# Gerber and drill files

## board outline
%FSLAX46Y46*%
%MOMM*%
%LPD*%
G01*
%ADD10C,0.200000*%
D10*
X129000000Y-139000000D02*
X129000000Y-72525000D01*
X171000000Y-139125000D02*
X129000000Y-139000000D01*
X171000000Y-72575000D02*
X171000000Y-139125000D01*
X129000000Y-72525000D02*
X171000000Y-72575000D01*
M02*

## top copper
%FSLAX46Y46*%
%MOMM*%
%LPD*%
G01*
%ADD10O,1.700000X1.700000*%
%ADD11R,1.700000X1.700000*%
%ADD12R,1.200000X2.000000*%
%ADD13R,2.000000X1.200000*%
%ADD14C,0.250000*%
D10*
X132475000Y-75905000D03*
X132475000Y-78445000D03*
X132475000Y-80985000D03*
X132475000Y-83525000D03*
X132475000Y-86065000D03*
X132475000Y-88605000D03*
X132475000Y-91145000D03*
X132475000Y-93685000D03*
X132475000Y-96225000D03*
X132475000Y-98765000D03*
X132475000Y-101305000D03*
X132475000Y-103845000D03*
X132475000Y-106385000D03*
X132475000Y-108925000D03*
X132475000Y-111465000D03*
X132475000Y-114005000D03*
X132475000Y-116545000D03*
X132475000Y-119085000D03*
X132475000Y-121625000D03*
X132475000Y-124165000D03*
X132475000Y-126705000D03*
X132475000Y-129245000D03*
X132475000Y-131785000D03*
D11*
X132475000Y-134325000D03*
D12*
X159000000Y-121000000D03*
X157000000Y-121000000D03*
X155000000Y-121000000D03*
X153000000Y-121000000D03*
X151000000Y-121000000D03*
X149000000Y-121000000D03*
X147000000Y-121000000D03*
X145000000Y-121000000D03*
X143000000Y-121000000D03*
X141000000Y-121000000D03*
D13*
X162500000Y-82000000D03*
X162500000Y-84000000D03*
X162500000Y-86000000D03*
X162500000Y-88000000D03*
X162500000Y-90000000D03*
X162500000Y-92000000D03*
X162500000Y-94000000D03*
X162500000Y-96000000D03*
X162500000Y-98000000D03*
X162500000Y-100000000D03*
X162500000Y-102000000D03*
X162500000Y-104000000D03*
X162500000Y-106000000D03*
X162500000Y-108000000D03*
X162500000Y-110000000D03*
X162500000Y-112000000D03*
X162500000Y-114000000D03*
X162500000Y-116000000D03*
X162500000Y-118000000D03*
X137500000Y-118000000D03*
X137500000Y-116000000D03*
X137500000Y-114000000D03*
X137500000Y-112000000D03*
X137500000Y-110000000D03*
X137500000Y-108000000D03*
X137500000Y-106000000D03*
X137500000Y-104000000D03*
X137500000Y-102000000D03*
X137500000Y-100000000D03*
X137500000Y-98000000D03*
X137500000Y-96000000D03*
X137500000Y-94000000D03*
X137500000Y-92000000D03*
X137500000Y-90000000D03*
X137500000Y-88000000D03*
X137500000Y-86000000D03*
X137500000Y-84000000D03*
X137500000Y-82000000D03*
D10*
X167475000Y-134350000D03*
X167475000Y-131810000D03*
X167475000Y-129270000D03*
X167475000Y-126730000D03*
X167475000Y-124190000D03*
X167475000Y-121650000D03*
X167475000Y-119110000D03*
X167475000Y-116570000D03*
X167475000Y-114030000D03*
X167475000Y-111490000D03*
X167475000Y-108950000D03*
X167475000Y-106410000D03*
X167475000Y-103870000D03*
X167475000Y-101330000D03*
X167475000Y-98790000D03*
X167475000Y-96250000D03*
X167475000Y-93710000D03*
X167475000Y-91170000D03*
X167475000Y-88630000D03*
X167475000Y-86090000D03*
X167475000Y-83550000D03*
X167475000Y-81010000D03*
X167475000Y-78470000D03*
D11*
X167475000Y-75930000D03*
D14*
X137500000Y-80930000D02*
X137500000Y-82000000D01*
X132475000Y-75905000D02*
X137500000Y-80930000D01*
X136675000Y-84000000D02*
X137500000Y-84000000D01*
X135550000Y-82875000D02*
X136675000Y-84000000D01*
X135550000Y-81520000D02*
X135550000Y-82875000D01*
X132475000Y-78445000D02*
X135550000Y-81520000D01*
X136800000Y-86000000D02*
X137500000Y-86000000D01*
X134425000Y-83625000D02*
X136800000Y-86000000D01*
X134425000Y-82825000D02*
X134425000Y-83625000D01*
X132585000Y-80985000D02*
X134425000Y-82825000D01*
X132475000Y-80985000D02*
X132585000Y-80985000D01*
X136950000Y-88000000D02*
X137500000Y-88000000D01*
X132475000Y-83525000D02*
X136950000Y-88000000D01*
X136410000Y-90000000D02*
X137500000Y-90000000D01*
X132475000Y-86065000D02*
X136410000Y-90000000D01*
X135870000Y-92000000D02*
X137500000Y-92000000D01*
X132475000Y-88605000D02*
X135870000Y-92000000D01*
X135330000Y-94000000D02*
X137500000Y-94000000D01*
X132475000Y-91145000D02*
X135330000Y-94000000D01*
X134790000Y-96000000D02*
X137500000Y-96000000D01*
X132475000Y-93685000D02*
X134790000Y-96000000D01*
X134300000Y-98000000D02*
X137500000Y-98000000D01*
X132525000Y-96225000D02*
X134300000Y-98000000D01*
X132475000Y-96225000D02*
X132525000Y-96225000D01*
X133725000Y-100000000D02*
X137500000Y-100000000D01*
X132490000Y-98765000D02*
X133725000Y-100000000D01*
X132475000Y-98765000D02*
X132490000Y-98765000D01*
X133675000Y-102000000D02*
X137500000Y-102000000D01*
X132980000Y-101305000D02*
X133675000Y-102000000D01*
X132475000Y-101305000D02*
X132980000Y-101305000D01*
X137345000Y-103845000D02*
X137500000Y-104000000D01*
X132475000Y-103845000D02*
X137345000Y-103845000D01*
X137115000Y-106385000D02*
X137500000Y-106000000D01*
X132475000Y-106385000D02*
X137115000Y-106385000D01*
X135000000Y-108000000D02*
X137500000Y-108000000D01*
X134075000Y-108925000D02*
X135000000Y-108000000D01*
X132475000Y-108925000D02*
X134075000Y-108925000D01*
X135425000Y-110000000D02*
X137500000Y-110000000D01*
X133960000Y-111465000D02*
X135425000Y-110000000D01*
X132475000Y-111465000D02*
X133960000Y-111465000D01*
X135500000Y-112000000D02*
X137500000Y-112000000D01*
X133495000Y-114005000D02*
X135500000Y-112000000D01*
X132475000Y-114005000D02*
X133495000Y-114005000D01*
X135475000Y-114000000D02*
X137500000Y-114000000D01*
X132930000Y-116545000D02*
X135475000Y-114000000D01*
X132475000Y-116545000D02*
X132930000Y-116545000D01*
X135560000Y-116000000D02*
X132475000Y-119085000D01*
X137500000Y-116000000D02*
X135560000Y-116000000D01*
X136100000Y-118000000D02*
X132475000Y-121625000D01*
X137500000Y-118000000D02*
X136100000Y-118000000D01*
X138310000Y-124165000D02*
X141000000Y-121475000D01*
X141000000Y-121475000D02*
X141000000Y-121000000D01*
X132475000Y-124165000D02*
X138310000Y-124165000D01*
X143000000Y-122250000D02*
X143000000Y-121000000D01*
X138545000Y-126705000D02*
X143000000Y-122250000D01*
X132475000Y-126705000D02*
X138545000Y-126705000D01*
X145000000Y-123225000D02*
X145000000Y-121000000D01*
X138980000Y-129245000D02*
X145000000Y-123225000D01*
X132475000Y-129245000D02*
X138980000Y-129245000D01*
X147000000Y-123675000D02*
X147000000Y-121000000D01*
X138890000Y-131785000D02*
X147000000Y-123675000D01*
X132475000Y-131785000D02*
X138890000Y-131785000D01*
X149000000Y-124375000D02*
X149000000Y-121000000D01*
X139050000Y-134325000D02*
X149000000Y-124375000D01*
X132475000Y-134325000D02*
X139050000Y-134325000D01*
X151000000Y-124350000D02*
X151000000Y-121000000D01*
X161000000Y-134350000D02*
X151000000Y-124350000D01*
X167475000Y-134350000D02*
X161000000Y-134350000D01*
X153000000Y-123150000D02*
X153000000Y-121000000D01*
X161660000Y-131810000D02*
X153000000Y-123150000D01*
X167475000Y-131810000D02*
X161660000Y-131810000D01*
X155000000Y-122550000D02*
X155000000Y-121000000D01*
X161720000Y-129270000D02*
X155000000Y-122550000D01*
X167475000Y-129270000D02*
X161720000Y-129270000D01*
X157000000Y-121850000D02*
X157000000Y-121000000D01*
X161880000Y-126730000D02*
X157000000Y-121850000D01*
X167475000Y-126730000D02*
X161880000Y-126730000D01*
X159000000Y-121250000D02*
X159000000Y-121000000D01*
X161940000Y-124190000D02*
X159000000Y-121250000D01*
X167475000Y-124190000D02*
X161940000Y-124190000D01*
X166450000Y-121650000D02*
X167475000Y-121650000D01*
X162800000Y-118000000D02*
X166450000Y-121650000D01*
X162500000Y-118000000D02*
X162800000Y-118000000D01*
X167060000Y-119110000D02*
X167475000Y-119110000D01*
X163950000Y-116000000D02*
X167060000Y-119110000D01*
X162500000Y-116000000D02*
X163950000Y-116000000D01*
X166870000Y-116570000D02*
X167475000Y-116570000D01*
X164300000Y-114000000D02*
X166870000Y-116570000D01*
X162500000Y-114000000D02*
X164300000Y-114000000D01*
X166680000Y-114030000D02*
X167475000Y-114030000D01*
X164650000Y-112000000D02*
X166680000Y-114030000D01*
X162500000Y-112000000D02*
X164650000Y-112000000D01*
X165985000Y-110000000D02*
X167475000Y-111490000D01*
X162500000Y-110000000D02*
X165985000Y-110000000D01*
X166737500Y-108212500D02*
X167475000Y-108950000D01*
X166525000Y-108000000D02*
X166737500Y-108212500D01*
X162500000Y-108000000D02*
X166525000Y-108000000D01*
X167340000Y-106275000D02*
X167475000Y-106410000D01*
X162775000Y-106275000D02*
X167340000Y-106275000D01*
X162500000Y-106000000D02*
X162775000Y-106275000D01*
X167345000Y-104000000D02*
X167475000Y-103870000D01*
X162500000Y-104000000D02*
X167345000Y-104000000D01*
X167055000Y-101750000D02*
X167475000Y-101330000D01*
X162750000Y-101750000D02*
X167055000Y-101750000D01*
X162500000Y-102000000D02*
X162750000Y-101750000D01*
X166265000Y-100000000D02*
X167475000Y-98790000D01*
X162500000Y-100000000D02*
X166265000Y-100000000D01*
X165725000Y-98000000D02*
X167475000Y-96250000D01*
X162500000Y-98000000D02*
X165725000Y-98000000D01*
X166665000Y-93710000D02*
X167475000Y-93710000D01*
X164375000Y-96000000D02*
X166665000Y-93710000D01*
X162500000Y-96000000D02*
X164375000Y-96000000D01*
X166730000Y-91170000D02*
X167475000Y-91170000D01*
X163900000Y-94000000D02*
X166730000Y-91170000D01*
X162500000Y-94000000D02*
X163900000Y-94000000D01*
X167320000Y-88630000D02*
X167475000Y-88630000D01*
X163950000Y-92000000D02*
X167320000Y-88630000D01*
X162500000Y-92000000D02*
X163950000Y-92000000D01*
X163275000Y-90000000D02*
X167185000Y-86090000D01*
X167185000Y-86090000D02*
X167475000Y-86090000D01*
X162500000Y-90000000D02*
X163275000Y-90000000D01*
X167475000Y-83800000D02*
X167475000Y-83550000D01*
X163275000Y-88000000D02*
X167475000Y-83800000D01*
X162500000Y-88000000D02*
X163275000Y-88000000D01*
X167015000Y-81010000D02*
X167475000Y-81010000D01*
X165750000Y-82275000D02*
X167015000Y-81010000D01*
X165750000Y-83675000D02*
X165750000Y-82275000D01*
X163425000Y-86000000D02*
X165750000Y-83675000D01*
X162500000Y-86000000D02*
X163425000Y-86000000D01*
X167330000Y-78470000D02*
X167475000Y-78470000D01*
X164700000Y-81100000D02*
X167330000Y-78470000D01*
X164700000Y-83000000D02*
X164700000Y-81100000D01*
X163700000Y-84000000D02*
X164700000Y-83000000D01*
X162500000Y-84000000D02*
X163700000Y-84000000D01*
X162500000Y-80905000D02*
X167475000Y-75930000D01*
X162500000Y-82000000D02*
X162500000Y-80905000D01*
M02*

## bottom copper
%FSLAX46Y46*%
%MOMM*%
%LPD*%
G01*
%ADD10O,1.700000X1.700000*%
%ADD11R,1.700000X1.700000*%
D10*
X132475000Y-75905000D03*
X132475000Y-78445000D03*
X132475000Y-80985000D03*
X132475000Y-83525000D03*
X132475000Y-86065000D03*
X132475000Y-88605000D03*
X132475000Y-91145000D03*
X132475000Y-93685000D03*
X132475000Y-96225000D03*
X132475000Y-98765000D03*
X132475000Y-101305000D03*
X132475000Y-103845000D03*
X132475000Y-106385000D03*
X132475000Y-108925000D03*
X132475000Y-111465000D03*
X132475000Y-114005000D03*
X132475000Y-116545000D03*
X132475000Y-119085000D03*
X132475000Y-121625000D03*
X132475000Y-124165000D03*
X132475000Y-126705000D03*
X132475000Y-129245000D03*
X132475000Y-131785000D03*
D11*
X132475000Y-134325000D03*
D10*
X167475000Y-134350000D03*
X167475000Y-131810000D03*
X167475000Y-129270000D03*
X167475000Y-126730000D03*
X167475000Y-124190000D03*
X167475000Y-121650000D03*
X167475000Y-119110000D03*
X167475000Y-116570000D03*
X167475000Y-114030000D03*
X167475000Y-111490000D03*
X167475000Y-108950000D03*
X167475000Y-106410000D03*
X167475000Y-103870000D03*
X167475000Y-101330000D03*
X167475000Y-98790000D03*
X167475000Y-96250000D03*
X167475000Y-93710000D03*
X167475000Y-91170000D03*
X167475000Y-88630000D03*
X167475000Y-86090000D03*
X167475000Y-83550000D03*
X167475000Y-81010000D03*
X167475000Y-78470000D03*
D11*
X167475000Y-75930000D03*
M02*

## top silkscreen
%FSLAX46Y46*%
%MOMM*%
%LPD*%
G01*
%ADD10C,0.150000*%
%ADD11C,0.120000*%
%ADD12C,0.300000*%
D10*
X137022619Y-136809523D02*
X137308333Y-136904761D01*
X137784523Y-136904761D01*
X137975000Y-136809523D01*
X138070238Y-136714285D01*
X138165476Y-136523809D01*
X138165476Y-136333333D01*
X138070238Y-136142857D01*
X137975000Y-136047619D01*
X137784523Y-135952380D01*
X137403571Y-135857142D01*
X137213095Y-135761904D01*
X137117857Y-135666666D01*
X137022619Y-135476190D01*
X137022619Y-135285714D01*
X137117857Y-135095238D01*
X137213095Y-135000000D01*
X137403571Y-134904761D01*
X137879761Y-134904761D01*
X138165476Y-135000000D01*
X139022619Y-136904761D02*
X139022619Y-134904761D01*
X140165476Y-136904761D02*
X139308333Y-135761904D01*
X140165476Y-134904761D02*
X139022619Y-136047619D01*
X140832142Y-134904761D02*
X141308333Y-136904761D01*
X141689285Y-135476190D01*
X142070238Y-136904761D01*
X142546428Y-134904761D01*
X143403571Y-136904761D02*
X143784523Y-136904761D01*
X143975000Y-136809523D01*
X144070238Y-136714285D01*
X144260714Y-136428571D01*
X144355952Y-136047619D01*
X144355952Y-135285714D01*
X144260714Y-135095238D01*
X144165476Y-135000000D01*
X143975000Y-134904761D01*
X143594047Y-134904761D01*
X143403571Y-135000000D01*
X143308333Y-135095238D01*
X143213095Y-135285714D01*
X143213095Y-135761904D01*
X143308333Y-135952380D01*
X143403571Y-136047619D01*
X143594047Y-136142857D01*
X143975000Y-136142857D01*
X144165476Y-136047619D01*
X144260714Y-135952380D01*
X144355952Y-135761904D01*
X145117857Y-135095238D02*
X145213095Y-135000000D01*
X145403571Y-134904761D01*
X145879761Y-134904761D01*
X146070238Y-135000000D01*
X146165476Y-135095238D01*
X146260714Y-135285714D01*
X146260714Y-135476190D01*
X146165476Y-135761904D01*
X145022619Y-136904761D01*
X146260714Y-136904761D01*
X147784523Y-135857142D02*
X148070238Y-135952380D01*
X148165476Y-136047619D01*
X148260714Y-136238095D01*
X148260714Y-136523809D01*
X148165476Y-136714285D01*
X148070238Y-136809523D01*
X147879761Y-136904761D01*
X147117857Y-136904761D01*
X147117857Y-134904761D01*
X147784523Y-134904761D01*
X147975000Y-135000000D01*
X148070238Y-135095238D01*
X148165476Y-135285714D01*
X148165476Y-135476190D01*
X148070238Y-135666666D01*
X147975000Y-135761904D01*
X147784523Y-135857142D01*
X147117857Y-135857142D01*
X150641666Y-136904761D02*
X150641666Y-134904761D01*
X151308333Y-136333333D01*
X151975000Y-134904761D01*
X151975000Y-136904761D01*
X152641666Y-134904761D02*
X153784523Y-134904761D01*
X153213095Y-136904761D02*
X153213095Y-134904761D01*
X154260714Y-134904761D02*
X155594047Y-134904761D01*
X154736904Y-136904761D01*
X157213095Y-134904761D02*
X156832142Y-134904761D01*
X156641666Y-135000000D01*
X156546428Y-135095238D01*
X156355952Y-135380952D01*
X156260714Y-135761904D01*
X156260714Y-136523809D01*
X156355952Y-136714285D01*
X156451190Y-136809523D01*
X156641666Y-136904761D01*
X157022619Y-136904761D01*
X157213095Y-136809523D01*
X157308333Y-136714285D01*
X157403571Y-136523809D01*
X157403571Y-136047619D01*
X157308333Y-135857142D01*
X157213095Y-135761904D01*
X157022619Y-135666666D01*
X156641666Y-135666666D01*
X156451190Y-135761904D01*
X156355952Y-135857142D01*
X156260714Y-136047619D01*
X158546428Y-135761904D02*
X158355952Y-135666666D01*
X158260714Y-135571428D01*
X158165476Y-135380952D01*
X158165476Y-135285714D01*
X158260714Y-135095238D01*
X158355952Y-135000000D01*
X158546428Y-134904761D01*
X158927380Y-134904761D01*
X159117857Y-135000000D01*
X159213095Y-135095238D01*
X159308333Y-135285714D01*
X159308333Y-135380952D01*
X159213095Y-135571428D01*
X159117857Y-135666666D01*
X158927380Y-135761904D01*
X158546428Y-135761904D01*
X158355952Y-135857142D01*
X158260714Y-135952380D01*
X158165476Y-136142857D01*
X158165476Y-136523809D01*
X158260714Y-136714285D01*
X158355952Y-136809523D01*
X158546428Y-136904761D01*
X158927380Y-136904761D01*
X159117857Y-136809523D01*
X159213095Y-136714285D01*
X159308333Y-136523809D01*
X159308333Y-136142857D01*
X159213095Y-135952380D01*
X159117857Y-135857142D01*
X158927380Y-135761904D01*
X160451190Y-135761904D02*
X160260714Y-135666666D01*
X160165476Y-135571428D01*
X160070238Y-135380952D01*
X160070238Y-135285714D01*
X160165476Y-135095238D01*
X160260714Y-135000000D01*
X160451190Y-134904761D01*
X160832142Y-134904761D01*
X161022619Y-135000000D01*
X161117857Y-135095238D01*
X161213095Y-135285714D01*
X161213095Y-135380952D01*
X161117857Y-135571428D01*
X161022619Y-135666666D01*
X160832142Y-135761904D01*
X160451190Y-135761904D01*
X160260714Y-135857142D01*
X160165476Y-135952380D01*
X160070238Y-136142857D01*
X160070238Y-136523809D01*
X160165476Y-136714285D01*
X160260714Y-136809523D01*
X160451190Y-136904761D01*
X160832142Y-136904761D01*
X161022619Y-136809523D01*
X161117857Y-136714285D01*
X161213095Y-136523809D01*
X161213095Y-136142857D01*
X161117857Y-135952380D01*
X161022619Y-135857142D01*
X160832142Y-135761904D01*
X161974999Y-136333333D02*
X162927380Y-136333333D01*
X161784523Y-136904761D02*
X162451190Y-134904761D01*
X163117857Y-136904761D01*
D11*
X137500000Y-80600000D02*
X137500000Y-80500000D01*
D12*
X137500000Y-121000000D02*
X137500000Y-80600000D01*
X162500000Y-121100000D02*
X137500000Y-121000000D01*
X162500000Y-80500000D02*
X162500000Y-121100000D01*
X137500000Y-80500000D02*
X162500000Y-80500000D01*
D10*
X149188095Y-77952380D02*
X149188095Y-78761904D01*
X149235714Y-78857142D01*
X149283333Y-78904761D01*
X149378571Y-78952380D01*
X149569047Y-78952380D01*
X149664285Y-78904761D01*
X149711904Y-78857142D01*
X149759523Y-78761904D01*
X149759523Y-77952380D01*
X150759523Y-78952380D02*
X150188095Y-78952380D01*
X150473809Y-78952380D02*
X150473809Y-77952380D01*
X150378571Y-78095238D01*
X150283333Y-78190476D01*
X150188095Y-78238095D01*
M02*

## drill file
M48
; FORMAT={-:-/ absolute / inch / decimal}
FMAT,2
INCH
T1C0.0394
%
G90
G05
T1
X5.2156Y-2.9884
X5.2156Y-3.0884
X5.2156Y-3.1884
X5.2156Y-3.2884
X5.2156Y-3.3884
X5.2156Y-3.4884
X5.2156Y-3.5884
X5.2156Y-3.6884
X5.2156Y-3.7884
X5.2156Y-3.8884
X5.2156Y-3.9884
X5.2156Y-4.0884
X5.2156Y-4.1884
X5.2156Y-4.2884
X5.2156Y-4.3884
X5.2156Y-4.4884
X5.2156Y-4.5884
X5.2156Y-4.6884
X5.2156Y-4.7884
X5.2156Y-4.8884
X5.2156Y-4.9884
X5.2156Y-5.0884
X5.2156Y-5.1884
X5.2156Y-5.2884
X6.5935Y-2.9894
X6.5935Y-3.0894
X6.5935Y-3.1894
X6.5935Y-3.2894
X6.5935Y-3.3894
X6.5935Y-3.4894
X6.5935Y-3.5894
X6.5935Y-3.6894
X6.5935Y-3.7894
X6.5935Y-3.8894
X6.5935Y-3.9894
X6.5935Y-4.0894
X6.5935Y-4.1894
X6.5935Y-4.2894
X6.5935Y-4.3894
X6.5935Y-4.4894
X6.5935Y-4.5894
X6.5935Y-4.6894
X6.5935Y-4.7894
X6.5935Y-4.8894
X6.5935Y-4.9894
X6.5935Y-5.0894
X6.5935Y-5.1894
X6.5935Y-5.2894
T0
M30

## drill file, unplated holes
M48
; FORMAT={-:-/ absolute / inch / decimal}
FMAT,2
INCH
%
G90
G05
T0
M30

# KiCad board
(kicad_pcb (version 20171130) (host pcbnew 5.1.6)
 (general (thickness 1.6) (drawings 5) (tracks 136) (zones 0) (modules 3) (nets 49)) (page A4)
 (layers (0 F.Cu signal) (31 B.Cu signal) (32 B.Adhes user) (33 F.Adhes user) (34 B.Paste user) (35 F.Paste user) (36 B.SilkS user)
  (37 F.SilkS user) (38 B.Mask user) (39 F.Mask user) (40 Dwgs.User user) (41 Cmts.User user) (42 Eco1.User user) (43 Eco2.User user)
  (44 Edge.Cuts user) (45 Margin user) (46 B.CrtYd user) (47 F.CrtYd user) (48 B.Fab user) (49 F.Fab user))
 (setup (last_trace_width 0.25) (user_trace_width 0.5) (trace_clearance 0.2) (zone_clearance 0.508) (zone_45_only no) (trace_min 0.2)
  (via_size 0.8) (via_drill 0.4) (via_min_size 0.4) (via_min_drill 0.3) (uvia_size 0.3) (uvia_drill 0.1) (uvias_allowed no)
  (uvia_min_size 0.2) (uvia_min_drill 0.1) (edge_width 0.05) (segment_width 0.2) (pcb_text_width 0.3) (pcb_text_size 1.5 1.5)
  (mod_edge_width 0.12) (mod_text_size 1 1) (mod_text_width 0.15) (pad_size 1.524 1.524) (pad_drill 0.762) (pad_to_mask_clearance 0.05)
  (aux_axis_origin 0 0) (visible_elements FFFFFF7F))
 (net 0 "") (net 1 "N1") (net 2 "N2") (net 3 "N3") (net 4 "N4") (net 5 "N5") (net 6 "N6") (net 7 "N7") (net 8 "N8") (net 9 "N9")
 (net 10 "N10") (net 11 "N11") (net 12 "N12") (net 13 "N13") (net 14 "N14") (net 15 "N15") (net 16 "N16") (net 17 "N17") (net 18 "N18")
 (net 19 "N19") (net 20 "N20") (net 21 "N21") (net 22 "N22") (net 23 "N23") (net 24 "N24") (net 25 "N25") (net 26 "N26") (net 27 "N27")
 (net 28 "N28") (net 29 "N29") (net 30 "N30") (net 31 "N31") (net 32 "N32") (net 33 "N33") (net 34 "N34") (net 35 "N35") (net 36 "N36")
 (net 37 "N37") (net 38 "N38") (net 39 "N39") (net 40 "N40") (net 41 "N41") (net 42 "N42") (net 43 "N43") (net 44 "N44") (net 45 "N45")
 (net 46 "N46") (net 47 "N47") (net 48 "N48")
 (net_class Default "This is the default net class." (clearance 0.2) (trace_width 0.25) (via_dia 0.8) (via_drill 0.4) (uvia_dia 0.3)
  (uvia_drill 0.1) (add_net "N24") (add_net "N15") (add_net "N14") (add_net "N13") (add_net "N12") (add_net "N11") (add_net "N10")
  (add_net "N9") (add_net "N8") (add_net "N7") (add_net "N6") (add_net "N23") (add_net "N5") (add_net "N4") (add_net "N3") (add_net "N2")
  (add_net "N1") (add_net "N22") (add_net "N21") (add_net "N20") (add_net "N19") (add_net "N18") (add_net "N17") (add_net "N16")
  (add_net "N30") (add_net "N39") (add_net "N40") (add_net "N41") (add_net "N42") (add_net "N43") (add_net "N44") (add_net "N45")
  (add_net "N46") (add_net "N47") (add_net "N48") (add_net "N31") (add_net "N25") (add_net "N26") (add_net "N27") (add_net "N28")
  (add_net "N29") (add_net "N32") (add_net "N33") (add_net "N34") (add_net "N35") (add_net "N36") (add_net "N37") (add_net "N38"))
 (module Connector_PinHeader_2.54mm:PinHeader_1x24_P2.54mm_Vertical (layer B.Cu) (at 132.475 134.325)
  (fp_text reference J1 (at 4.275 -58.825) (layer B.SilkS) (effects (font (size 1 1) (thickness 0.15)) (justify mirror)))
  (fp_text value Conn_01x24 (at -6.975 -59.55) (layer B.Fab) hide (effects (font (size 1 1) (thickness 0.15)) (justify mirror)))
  (pad 24 thru_hole oval (at 0 -58.42) (size 1.7 1.7) (drill 1) (layers *.Cu *.Mask) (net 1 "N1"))
  (pad 23 thru_hole oval (at 0 -55.88) (size 1.7 1.7) (drill 1) (layers *.Cu *.Mask) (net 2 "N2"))
  (pad 22 thru_hole oval (at 0 -53.34) (size 1.7 1.7) (drill 1) (layers *.Cu *.Mask) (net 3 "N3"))
  (pad 21 thru_hole oval (at 0 -50.8) (size 1.7 1.7) (drill 1) (layers *.Cu *.Mask) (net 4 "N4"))
  (pad 20 thru_hole oval (at 0 -48.26) (size 1.7 1.7) (drill 1) (layers *.Cu *.Mask) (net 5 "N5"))
  (pad 19 thru_hole oval (at 0 -45.72) (size 1.7 1.7) (drill 1) (layers *.Cu *.Mask) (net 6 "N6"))
  (pad 18 thru_hole oval (at 0 -43.18) (size 1.7 1.7) (drill 1) (layers *.Cu *.Mask) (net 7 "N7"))
  (pad 17 thru_hole oval (at 0 -40.64) (size 1.7 1.7) (drill 1) (layers *.Cu *.Mask) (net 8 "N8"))
  (pad 16 thru_hole oval (at 0 -38.1) (size 1.7 1.7) (drill 1) (layers *.Cu *.Mask) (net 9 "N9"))
  (pad 15 thru_hole oval (at 0 -35.56) (size 1.7 1.7) (drill 1) (layers *.Cu *.Mask) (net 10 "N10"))
  (pad 14 thru_hole oval (at 0 -33.02) (size 1.7 1.7) (drill 1) (layers *.Cu *.Mask) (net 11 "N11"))
  (pad 13 thru_hole oval (at 0 -30.48) (size 1.7 1.7) (drill 1) (layers *.Cu *.Mask) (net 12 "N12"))
  (pad 12 thru_hole oval (at 0 -27.94) (size 1.7 1.7) (drill 1) (layers *.Cu *.Mask) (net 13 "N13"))
  (pad 11 thru_hole oval (at 0 -25.4) (size 1.7 1.7) (drill 1) (layers *.Cu *.Mask) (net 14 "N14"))
  (pad 10 thru_hole oval (at 0 -22.86) (size 1.7 1.7) (drill 1) (layers *.Cu *.Mask) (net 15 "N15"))
  (pad 9 thru_hole oval (at 0 -20.32) (size 1.7 1.7) (drill 1) (layers *.Cu *.Mask) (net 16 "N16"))
  (pad 8 thru_hole oval (at 0 -17.78) (size 1.7 1.7) (drill 1) (layers *.Cu *.Mask) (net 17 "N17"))
  (pad 7 thru_hole oval (at 0 -15.24) (size 1.7 1.7) (drill 1) (layers *.Cu *.Mask) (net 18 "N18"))
  (pad 6 thru_hole oval (at 0 -12.7) (size 1.7 1.7) (drill 1) (layers *.Cu *.Mask) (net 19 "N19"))
  (pad 5 thru_hole oval (at 0 -10.16) (size 1.7 1.7) (drill 1) (layers *.Cu *.Mask) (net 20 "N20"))
  (pad 4 thru_hole oval (at 0 -7.62) (size 1.7 1.7) (drill 1) (layers *.Cu *.Mask) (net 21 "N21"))
  (pad 3 thru_hole oval (at 0 -5.08) (size 1.7 1.7) (drill 1) (layers *.Cu *.Mask) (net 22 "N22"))
  (pad 2 thru_hole oval (at 0 -2.54) (size 1.7 1.7) (drill 1) (layers *.Cu *.Mask) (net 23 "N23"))
  (pad 1 thru_hole rect (at 0 0) (size 1.7 1.7) (drill 1) (layers *.Cu *.Mask) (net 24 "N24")))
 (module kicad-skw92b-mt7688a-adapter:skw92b (layer F.Cu) (at 150 100)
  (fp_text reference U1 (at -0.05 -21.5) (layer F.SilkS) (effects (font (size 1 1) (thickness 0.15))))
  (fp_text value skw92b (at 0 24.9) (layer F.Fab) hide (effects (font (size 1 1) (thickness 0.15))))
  (fp_line (start -12.5 -19.4) (end -12.5 -19.5) (layer F.SilkS) (width 0.12))
  (fp_line (start -12.5 21) (end -12.5 -19.4) (layer F.SilkS) (width 0.3))
  (fp_line (start 12.5 21.1) (end -12.5 21) (layer F.SilkS) (width 0.3))
  (fp_line (start 12.5 -19.5) (end 12.5 21.1) (layer F.SilkS) (width 0.3))
  (fp_line (start -12.5 -19.5) (end 12.5 -19.5) (layer F.SilkS) (width 0.3))
  (pad 29 smd rect (at 9 21) (size 1.2 2) (layers F.Cu F.Paste F.Mask) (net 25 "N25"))
  (pad 28 smd rect (at 7 21) (size 1.2 2) (layers F.Cu F.Paste F.Mask) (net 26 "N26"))
  (pad 27 smd rect (at 5 21) (size 1.2 2) (layers F.Cu F.Paste F.Mask) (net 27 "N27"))
  (pad 26 smd rect (at 3 21) (size 1.2 2) (layers F.Cu F.Paste F.Mask) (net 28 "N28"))
  (pad 25 smd rect (at 1 21) (size 1.2 2) (layers F.Cu F.Paste F.Mask) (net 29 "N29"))
  (pad 24 smd rect (at -1 21) (size 1.2 2) (layers F.Cu F.Paste F.Mask) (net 24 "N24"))
  (pad 23 smd rect (at -3 21) (size 1.2 2) (layers F.Cu F.Paste F.Mask) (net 23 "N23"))
  (pad 22 smd rect (at -5 21) (size 1.2 2) (layers F.Cu F.Paste F.Mask) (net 22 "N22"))
  (pad 21 smd rect (at -7 21) (size 1.2 2) (layers F.Cu F.Paste F.Mask) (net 21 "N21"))
  (pad 20 smd rect (at -9 21) (size 1.2 2) (layers F.Cu F.Paste F.Mask) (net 20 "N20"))
  (pad 48 smd rect (at 12.5 -18) (size 2 1.2) (layers F.Cu F.Paste F.Mask) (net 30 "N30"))
  (pad 47 smd rect (at 12.5 -16) (size 2 1.2) (layers F.Cu F.Paste F.Mask) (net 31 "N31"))
  (pad 46 smd rect (at 12.5 -14) (size 2 1.2) (layers F.Cu F.Paste F.Mask) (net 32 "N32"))
  (pad 45 smd rect (at 12.5 -12) (size 2 1.2) (layers F.Cu F.Paste F.Mask) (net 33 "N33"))
  (pad 44 smd rect (at 12.5 -10) (size 2 1.2) (layers F.Cu F.Paste F.Mask) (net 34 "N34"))
  (pad 43 smd rect (at 12.5 -8) (size 2 1.2) (layers F.Cu F.Paste F.Mask) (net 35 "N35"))
  (pad 42 smd rect (at 12.5 -6) (size 2 1.2) (layers F.Cu F.Paste F.Mask) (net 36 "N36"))
  (pad 41 smd rect (at 12.5 -4) (size 2 1.2) (layers F.Cu F.Paste F.Mask) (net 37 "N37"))
  (pad 40 smd rect (at 12.5 -2) (size 2 1.2) (layers F.Cu F.Paste F.Mask) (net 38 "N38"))
  (pad 39 smd rect (at 12.5 0) (size 2 1.2) (layers F.Cu F.Paste F.Mask) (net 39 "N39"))
  (pad 38 smd rect (at 12.5 2) (size 2 1.2) (layers F.Cu F.Paste F.Mask) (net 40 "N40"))
  (pad 37 smd rect (at 12.5 4) (size 2 1.2) (layers F.Cu F.Paste F.Mask) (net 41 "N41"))
  (pad 36 smd rect (at 12.5 6) (size 2 1.2) (layers F.Cu F.Paste F.Mask) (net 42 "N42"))
  (pad 35 smd rect (at 12.5 8) (size 2 1.2) (layers F.Cu F.Paste F.Mask) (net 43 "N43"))
  (pad 34 smd rect (at 12.5 10) (size 2 1.2) (layers F.Cu F.Paste F.Mask) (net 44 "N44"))
  (pad 33 smd rect (at 12.5 12) (size 2 1.2) (layers F.Cu F.Paste F.Mask) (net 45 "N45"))
  (pad 32 smd rect (at 12.5 14) (size 2 1.2) (layers F.Cu F.Paste F.Mask) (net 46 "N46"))
  (pad 31 smd rect (at 12.5 16) (size 2 1.2) (layers F.Cu F.Paste F.Mask) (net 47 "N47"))
  (pad 30 smd rect (at 12.5 18) (size 2 1.2) (layers F.Cu F.Paste F.Mask) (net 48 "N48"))
  (pad 19 smd rect (at -12.5 18) (size 2 1.2) (layers F.Cu F.Paste F.Mask) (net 19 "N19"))
  (pad 18 smd rect (at -12.5 16) (size 2 1.2) (layers F.Cu F.Paste F.Mask) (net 18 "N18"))
  (pad 17 smd rect (at -12.5 14) (size 2 1.2) (layers F.Cu F.Paste F.Mask) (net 17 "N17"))
  (pad 16 smd rect (at -12.5 12) (size 2 1.2) (layers F.Cu F.Paste F.Mask) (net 16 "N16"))
  (pad 15 smd rect (at -12.5 10) (size 2 1.2) (layers F.Cu F.Paste F.Mask) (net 15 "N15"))
  (pad 14 smd rect (at -12.5 8) (size 2 1.2) (layers F.Cu F.Paste F.Mask) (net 14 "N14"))
  (pad 13 smd rect (at -12.5 6) (size 2 1.2) (layers F.Cu F.Paste F.Mask) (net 13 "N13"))
  (pad 12 smd rect (at -12.5 4) (size 2 1.2) (layers F.Cu F.Paste F.Mask) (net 12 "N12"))
  (pad 11 smd rect (at -12.5 2) (size 2 1.2) (layers F.Cu F.Paste F.Mask) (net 11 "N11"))
  (pad 10 smd rect (at -12.5 0) (size 2 1.2) (layers F.Cu F.Paste F.Mask) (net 10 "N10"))
  (pad 9 smd rect (at -12.5 -2) (size 2 1.2) (layers F.Cu F.Paste F.Mask) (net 9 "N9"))
  (pad 8 smd rect (at -12.5 -4) (size 2 1.2) (layers F.Cu F.Paste F.Mask) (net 8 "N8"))
  (pad 7 smd rect (at -12.5 -6) (size 2 1.2) (layers F.Cu F.Paste F.Mask) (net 7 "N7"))
  (pad 6 smd rect (at -12.5 -8) (size 2 1.2) (layers F.Cu F.Paste F.Mask) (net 6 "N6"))
  (pad 5 smd rect (at -12.5 -10) (size 2 1.2) (layers F.Cu F.Paste F.Mask) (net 5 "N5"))
  (pad 4 smd rect (at -12.5 -12) (size 2 1.2) (layers F.Cu F.Paste F.Mask) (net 4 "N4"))
  (pad 3 smd rect (at -12.5 -14) (size 2 1.2) (layers F.Cu F.Paste F.Mask) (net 3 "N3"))
  (pad 2 smd rect (at -12.5 -16) (size 2 1.2) (layers F.Cu F.Paste F.Mask) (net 2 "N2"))
  (pad 1 smd rect (at -12.5 -18) (size 2 1.2) (layers F.Cu F.Paste F.Mask) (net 1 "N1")))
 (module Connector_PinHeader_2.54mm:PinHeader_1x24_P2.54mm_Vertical (layer B.Cu) (at 167.475 75.93 180)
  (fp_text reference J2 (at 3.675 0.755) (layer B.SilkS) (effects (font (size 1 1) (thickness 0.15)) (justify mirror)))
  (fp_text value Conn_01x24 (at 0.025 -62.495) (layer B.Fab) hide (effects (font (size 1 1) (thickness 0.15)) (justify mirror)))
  (pad 24 thru_hole oval (at 0 -58.42 180) (size 1.7 1.7) (drill 1) (layers *.Cu *.Mask) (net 29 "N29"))
  (pad 23 thru_hole oval (at 0 -55.88 180) (size 1.7 1.7) (drill 1) (layers *.Cu *.Mask) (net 28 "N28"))
  (pad 22 thru_hole oval (at 0 -53.34 180) (size 1.7 1.7) (drill 1) (layers *.Cu *.Mask) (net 27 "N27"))
  (pad 21 thru_hole oval (at 0 -50.8 180) (size 1.7 1.7) (drill 1) (layers *.Cu *.Mask) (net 26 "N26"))
  (pad 20 thru_hole oval (at 0 -48.26 180) (size 1.7 1.7) (drill 1) (layers *.Cu *.Mask) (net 25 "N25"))
  (pad 19 thru_hole oval (at 0 -45.72 180) (size 1.7 1.7) (drill 1) (layers *.Cu *.Mask) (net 48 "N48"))
  (pad 18 thru_hole oval (at 0 -43.18 180) (size 1.7 1.7) (drill 1) (layers *.Cu *.Mask) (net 47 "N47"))
  (pad 17 thru_hole oval (at 0 -40.64 180) (size 1.7 1.7) (drill 1) (layers *.Cu *.Mask) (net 46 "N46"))
  (pad 16 thru_hole oval (at 0 -38.1 180) (size 1.7 1.7) (drill 1) (layers *.Cu *.Mask) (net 45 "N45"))
  (pad 15 thru_hole oval (at 0 -35.56 180) (size 1.7 1.7) (drill 1) (layers *.Cu *.Mask) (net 44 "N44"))
  (pad 14 thru_hole oval (at 0 -33.02 180) (size 1.7 1.7) (drill 1) (layers *.Cu *.Mask) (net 43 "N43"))
  (pad 13 thru_hole oval (at 0 -30.48 180) (size 1.7 1.7) (drill 1) (layers *.Cu *.Mask) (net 42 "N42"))
  (pad 12 thru_hole oval (at 0 -27.94 180) (size 1.7 1.7) (drill 1) (layers *.Cu *.Mask) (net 41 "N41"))
  (pad 11 thru_hole oval (at 0 -25.4 180) (size 1.7 1.7) (drill 1) (layers *.Cu *.Mask) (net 40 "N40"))
  (pad 10 thru_hole oval (at 0 -22.86 180) (size 1.7 1.7) (drill 1) (layers *.Cu *.Mask) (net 39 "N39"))
  (pad 9 thru_hole oval (at 0 -20.32 180) (size 1.7 1.7) (drill 1) (layers *.Cu *.Mask) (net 38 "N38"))
  (pad 8 thru_hole oval (at 0 -17.78 180) (size 1.7 1.7) (drill 1) (layers *.Cu *.Mask) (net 37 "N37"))
  (pad 7 thru_hole oval (at 0 -15.24 180) (size 1.7 1.7) (drill 1) (layers *.Cu *.Mask) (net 36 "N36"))
  (pad 6 thru_hole oval (at 0 -12.7 180) (size 1.7 1.7) (drill 1) (layers *.Cu *.Mask) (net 35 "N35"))
  (pad 5 thru_hole oval (at 0 -10.16 180) (size 1.7 1.7) (drill 1) (layers *.Cu *.Mask) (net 34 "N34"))
  (pad 4 thru_hole oval (at 0 -7.62 180) (size 1.7 1.7) (drill 1) (layers *.Cu *.Mask) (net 33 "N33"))
  (pad 3 thru_hole oval (at 0 -5.08 180) (size 1.7 1.7) (drill 1) (layers *.Cu *.Mask) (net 32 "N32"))
  (pad 2 thru_hole oval (at 0 -2.54 180) (size 1.7 1.7) (drill 1) (layers *.Cu *.Mask) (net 31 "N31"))
  (pad 1 thru_hole rect (at 0 0 180) (size 1.7 1.7) (drill 1) (layers *.Cu *.Mask) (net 30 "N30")))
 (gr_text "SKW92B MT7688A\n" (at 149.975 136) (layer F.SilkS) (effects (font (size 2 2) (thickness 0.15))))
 (gr_line (start 129 139) (end 129 72.525) (layer Edge.Cuts) (width 0.2))
 (gr_line (start 171 139.125) (end 129 139) (layer Edge.Cuts) (width 0.2))
 (gr_line (start 171 72.575) (end 171 139.125) (layer Edge.Cuts) (width 0.2))
 (gr_line (start 129 72.525) (end 171 72.575) (layer Edge.Cuts) (width 0.2))
 (segment (start 137.5 80.93) (end 137.5 82) (width 0.25) (layer F.Cu) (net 1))
 (segment (start 132.475 75.905) (end 137.5 80.93) (width 0.25) (layer F.Cu) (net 1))
 (segment (start 136.675 84) (end 137.5 84) (width 0.25) (layer F.Cu) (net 2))
 (segment (start 135.55 82.875) (end 136.675 84) (width 0.25) (layer F.Cu) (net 2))
 (segment (start 135.55 81.52) (end 135.55 82.875) (width 0.25) (layer F.Cu) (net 2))
 (segment (start 132.475 78.445) (end 135.55 81.52) (width 0.25) (layer F.Cu) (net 2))
 (segment (start 136.8 86) (end 137.5 86) (width 0.25) (layer F.Cu) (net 3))
 (segment (start 134.425 83.625) (end 136.8 86) (width 0.25) (layer F.Cu) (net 3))
 (segment (start 134.425 82.825) (end 134.425 83.625) (width 0.25) (layer F.Cu) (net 3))
 (segment (start 132.585 80.985) (end 134.425 82.825) (width 0.25) (layer F.Cu) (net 3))
 (segment (start 132.475 80.985) (end 132.585 80.985) (width 0.25) (layer F.Cu) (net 3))
 (segment (start 136.95 88) (end 137.5 88) (width 0.25) (layer F.Cu) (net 4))
 (segment (start 132.475 83.525) (end 136.95 88) (width 0.25) (layer F.Cu) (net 4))
 (segment (start 136.41 90) (end 137.5 90) (width 0.25) (layer F.Cu) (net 5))
 (segment (start 132.475 86.065) (end 136.41 90) (width 0.25) (layer F.Cu) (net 5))
 (segment (start 135.87 92) (end 137.5 92) (width 0.25) (layer F.Cu) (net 6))
 (segment (start 132.475 88.605) (end 135.87 92) (width 0.25) (layer F.Cu) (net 6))
 (segment (start 135.33 94) (end 137.5 94) (width 0.25) (layer F.Cu) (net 7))
 (segment (start 132.475 91.145) (end 135.33 94) (width 0.25) (layer F.Cu) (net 7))
 (segment (start 134.79 96) (end 137.5 96) (width 0.25) (layer F.Cu) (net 8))
 (segment (start 132.475 93.685) (end 134.79 96) (width 0.25) (layer F.Cu) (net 8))
 (segment (start 134.3 98) (end 137.5 98) (width 0.25) (layer F.Cu) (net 9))
 (segment (start 132.525 96.225) (end 134.3 98) (width 0.25) (layer F.Cu) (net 9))
 (segment (start 132.475 96.225) (end 132.525 96.225) (width 0.25) (layer F.Cu) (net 9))
 (segment (start 133.725 100) (end 137.5 100) (width 0.25) (layer F.Cu) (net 10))
 (segment (start 132.49 98.765) (end 133.725 100) (width 0.25) (layer F.Cu) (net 10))
 (segment (start 132.475 98.765) (end 132.49 98.765) (width 0.25) (layer F.Cu) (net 10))
 (segment (start 133.675 102) (end 137.5 102) (width 0.25) (layer F.Cu) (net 11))
 (segment (start 132.98 101.305) (end 133.675 102) (width 0.25) (layer F.Cu) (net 11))
 (segment (start 132.475 101.305) (end 132.98 101.305) (width 0.25) (layer F.Cu) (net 11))
 (segment (start 137.345 103.845) (end 137.5 104) (width 0.25) (layer F.Cu) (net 12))
 (segment (start 132.475 103.845) (end 137.345 103.845) (width 0.25) (layer F.Cu) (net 12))
 (segment (start 137.115 106.385) (end 137.5 106) (width 0.25) (layer F.Cu) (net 13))
 (segment (start 132.475 106.385) (end 137.115 106.385) (width 0.25) (layer F.Cu) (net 13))
 (segment (start 135 108) (end 137.5 108) (width 0.25) (layer F.Cu) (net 14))
 (segment (start 134.075 108.925) (end 135 108) (width 0.25) (layer F.Cu) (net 14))
 (segment (start 132.475 108.925) (end 134.075 108.925) (width 0.25) (layer F.Cu) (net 14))
 (segment (start 135.425 110) (end 137.5 110) (width 0.25) (layer F.Cu) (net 15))
 (segment (start 133.96 111.465) (end 135.425 110) (width 0.25) (layer F.Cu) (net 15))
 (segment (start 132.475 111.465) (end 133.96 111.465) (width 0.25) (layer F.Cu) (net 15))
 (segment (start 135.5 112) (end 137.5 112) (width 0.25) (layer F.Cu) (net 16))
 (segment (start 133.495 114.005) (end 135.5 112) (width 0.25) (layer F.Cu) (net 16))
 (segment (start 132.475 114.005) (end 133.495 114.005) (width 0.25) (layer F.Cu) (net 16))
 (segment (start 135.475 114) (end 137.5 114) (width 0.25) (layer F.Cu) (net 17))
 (segment (start 132.93 116.545) (end 135.475 114) (width 0.25) (layer F.Cu) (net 17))
 (segment (start 132.475 116.545) (end 132.93 116.545) (width 0.25) (layer F.Cu) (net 17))
 (segment (start 135.56 116) (end 132.475 119.085) (width 0.25) (layer F.Cu) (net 18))
 (segment (start 137.5 116) (end 135.56 116) (width 0.25) (layer F.Cu) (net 18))
 (segment (start 136.1 118) (end 132.475 121.625) (width 0.25) (layer F.Cu) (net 19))
 (segment (start 137.5 118) (end 136.1 118) (width 0.25) (layer F.Cu) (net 19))
 (segment (start 138.31 124.165) (end 141 121.475) (width 0.25) (layer F.Cu) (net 20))
 (segment (start 141 121.475) (end 141 121) (width 0.25) (layer F.Cu) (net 20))
 (segment (start 132.475 124.165) (end 138.31 124.165) (width 0.25) (layer F.Cu) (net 20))
 (segment (start 143 122.25) (end 143 121) (width 0.25) (layer F.Cu) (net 21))
 (segment (start 138.545 126.705) (end 143 122.25) (width 0.25) (layer F.Cu) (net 21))
 (segment (start 132.475 126.705) (end 138.545 126.705) (width 0.25) (layer F.Cu) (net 21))
 (segment (start 145 123.225) (end 145 121) (width 0.25) (layer F.Cu) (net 22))
 (segment (start 138.98 129.245) (end 145 123.225) (width 0.25) (layer F.Cu) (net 22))
 (segment (start 132.475 129.245) (end 138.98 129.245) (width 0.25) (layer F.Cu) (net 22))
 (segment (start 147 123.675) (end 147 121) (width 0.25) (layer F.Cu) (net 23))
 (segment (start 138.89 131.785) (end 147 123.675) (width 0.25) (layer F.Cu) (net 23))
 (segment (start 132.475 131.785) (end 138.89 131.785) (width 0.25) (layer F.Cu) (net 23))
 (segment (start 149 124.375) (end 149 121) (width 0.25) (layer F.Cu) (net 24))
 (segment (start 139.05 134.325) (end 149 124.375) (width 0.25) (layer F.Cu) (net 24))
 (segment (start 132.475 134.325) (end 139.05 134.325) (width 0.25) (layer F.Cu) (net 24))
 (segment (start 151 124.35) (end 151 121) (width 0.25) (layer F.Cu) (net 29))
 (segment (start 161 134.35) (end 151 124.35) (width 0.25) (layer F.Cu) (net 29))
 (segment (start 167.475 134.35) (end 161 134.35) (width 0.25) (layer F.Cu) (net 29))
 (segment (start 153 123.15) (end 153 121) (width 0.25) (layer F.Cu) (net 28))
 (segment (start 161.66 131.81) (end 153 123.15) (width 0.25) (layer F.Cu) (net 28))
 (segment (start 167.475 131.81) (end 161.66 131.81) (width 0.25) (layer F.Cu) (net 28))
 (segment (start 155 122.55) (end 155 121) (width 0.25) (layer F.Cu) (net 27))
 (segment (start 161.72 129.27) (end 155 122.55) (width 0.25) (layer F.Cu) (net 27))
 (segment (start 167.475 129.27) (end 161.72 129.27) (width 0.25) (layer F.Cu) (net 27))
 (segment (start 157 121.85) (end 157 121) (width 0.25) (layer F.Cu) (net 26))
 (segment (start 161.88 126.73) (end 157 121.85) (width 0.25) (layer F.Cu) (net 26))
 (segment (start 167.475 126.73) (end 161.88 126.73) (width 0.25) (layer F.Cu) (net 26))
 (segment (start 159 121.25) (end 159 121) (width 0.25) (layer F.Cu) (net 25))
 (segment (start 161.94 124.19) (end 159 121.25) (width 0.25) (layer F.Cu) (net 25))
 (segment (start 167.475 124.19) (end 161.94 124.19) (width 0.25) (layer F.Cu) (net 25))
 (segment (start 166.45 121.65) (end 167.475 121.65) (width 0.25) (layer F.Cu) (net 48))
 (segment (start 162.8 118) (end 166.45 121.65) (width 0.25) (layer F.Cu) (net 48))
 (segment (start 162.5 118) (end 162.8 118) (width 0.25) (layer F.Cu) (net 48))
 (segment (start 167.06 119.11) (end 167.475 119.11) (width 0.25) (layer F.Cu) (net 47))
 (segment (start 163.95 116) (end 167.06 119.11) (width 0.25) (layer F.Cu) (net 47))
 (segment (start 162.5 116) (end 163.95 116) (width 0.25) (layer F.Cu) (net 47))
 (segment (start 166.87 116.57) (end 167.475 116.57) (width 0.25) (layer F.Cu) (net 46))
 (segment (start 164.3 114) (end 166.87 116.57) (width 0.25) (layer F.Cu) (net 46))
 (segment (start 162.5 114) (end 164.3 114) (width 0.25) (layer F.Cu) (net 46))
 (segment (start 166.68 114.03) (end 167.475 114.03) (width 0.25) (layer F.Cu) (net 45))
 (segment (start 164.65 112) (end 166.68 114.03) (width 0.25) (layer F.Cu) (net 45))
 (segment (start 162.5 112) (end 164.65 112) (width 0.25) (layer F.Cu) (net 45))
 (segment (start 165.985 110) (end 167.475 111.49) (width 0.25) (layer F.Cu) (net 44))
 (segment (start 162.5 110) (end 165.985 110) (width 0.25) (layer F.Cu) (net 44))
 (segment (start 166.7375 108.2125) (end 167.475 108.95) (width 0.25) (layer F.Cu) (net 43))
 (segment (start 166.525 108) (end 166.7375 108.2125) (width 0.25) (layer F.Cu) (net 43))
 (segment (start 162.5 108) (end 166.525 108) (width 0.25) (layer F.Cu) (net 43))
 (segment (start 167.34 106.275) (end 167.475 106.41) (width 0.25) (layer F.Cu) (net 42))
 (segment (start 162.775 106.275) (end 167.34 106.275) (width 0.25) (layer F.Cu) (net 42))
 (segment (start 162.5 106) (end 162.775 106.275) (width 0.25) (layer F.Cu) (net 42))
 (segment (start 167.345 104) (end 167.475 103.87) (width 0.25) (layer F.Cu) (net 41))
 (segment (start 162.5 104) (end 167.345 104) (width 0.25) (layer F.Cu) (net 41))
 (segment (start 167.055 101.75) (end 167.475 101.33) (width 0.25) (layer F.Cu) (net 40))
 (segment (start 162.75 101.75) (end 167.055 101.75) (width 0.25) (layer F.Cu) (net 40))
 (segment (start 162.5 102) (end 162.75 101.75) (width 0.25) (layer F.Cu) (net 40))
 (segment (start 166.265 100) (end 167.475 98.79) (width 0.25) (layer F.Cu) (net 39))
 (segment (start 162.5 100) (end 166.265 100) (width 0.25) (layer F.Cu) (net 39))
 (segment (start 165.725 98) (end 167.475 96.25) (width 0.25) (layer F.Cu) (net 38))
 (segment (start 162.5 98) (end 165.725 98) (width 0.25) (layer F.Cu) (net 38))
 (segment (start 166.665 93.71) (end 167.475 93.71) (width 0.25) (layer F.Cu) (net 37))
 (segment (start 164.375 96) (end 166.665 93.71) (width 0.25) (layer F.Cu) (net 37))
 (segment (start 162.5 96) (end 164.375 96) (width 0.25) (layer F.Cu) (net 37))
 (segment (start 166.73 91.17) (end 167.475 91.17) (width 0.25) (layer F.Cu) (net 36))
 (segment (start 163.9 94) (end 166.73 91.17) (width 0.25) (layer F.Cu) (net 36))
 (segment (start 162.5 94) (end 163.9 94) (width 0.25) (layer F.Cu) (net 36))
 (segment (start 167.32 88.63) (end 167.475 88.63) (width 0.25) (layer F.Cu) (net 35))
 (segment (start 163.95 92) (end 167.32 88.63) (width 0.25) (layer F.Cu) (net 35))
 (segment (start 162.5 92) (end 163.95 92) (width 0.25) (layer F.Cu) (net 35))
 (segment (start 163.275 90) (end 167.185 86.09) (width 0.25) (layer F.Cu) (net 34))
 (segment (start 167.185 86.09) (end 167.475 86.09) (width 0.25) (layer F.Cu) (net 34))
 (segment (start 162.5 90) (end 163.275 90) (width 0.25) (layer F.Cu) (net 34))
 (segment (start 167.475 83.8) (end 167.475 83.55) (width 0.25) (layer F.Cu) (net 33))
 (segment (start 163.275 88) (end 167.475 83.8) (width 0.25) (layer F.Cu) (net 33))
 (segment (start 162.5 88) (end 163.275 88) (width 0.25) (layer F.Cu) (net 33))
 (segment (start 167.015 81.01) (end 167.475 81.01) (width 0.25) (layer F.Cu) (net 32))
 (segment (start 165.75 82.275) (end 167.015 81.01) (width 0.25) (layer F.Cu) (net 32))
 (segment (start 165.75 83.675) (end 165.75 82.275) (width 0.25) (layer F.Cu) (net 32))
 (segment (start 163.425 86) (end 165.75 83.675) (width 0.25) (layer F.Cu) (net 32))
 (segment (start 162.5 86) (end 163.425 86) (width 0.25) (layer F.Cu) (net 32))
 (segment (start 167.33 78.47) (end 167.475 78.47) (width 0.25) (layer F.Cu) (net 31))
 (segment (start 164.7 81.1) (end 167.33 78.47) (width 0.25) (layer F.Cu) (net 31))
 (segment (start 164.7 83) (end 164.7 81.1) (width 0.25) (layer F.Cu) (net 31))
 (segment (start 163.7 84) (end 164.7 83) (width 0.25) (layer F.Cu) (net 31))
 (segment (start 162.5 84) (end 163.7 84) (width 0.25) (layer F.Cu) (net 31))
 (segment (start 162.5 80.905) (end 167.475 75.93) (width 0.25) (layer F.Cu) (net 30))
 (segment (start 162.5 82) (end 162.5 80.905) (width 0.25) (layer F.Cu) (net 30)))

